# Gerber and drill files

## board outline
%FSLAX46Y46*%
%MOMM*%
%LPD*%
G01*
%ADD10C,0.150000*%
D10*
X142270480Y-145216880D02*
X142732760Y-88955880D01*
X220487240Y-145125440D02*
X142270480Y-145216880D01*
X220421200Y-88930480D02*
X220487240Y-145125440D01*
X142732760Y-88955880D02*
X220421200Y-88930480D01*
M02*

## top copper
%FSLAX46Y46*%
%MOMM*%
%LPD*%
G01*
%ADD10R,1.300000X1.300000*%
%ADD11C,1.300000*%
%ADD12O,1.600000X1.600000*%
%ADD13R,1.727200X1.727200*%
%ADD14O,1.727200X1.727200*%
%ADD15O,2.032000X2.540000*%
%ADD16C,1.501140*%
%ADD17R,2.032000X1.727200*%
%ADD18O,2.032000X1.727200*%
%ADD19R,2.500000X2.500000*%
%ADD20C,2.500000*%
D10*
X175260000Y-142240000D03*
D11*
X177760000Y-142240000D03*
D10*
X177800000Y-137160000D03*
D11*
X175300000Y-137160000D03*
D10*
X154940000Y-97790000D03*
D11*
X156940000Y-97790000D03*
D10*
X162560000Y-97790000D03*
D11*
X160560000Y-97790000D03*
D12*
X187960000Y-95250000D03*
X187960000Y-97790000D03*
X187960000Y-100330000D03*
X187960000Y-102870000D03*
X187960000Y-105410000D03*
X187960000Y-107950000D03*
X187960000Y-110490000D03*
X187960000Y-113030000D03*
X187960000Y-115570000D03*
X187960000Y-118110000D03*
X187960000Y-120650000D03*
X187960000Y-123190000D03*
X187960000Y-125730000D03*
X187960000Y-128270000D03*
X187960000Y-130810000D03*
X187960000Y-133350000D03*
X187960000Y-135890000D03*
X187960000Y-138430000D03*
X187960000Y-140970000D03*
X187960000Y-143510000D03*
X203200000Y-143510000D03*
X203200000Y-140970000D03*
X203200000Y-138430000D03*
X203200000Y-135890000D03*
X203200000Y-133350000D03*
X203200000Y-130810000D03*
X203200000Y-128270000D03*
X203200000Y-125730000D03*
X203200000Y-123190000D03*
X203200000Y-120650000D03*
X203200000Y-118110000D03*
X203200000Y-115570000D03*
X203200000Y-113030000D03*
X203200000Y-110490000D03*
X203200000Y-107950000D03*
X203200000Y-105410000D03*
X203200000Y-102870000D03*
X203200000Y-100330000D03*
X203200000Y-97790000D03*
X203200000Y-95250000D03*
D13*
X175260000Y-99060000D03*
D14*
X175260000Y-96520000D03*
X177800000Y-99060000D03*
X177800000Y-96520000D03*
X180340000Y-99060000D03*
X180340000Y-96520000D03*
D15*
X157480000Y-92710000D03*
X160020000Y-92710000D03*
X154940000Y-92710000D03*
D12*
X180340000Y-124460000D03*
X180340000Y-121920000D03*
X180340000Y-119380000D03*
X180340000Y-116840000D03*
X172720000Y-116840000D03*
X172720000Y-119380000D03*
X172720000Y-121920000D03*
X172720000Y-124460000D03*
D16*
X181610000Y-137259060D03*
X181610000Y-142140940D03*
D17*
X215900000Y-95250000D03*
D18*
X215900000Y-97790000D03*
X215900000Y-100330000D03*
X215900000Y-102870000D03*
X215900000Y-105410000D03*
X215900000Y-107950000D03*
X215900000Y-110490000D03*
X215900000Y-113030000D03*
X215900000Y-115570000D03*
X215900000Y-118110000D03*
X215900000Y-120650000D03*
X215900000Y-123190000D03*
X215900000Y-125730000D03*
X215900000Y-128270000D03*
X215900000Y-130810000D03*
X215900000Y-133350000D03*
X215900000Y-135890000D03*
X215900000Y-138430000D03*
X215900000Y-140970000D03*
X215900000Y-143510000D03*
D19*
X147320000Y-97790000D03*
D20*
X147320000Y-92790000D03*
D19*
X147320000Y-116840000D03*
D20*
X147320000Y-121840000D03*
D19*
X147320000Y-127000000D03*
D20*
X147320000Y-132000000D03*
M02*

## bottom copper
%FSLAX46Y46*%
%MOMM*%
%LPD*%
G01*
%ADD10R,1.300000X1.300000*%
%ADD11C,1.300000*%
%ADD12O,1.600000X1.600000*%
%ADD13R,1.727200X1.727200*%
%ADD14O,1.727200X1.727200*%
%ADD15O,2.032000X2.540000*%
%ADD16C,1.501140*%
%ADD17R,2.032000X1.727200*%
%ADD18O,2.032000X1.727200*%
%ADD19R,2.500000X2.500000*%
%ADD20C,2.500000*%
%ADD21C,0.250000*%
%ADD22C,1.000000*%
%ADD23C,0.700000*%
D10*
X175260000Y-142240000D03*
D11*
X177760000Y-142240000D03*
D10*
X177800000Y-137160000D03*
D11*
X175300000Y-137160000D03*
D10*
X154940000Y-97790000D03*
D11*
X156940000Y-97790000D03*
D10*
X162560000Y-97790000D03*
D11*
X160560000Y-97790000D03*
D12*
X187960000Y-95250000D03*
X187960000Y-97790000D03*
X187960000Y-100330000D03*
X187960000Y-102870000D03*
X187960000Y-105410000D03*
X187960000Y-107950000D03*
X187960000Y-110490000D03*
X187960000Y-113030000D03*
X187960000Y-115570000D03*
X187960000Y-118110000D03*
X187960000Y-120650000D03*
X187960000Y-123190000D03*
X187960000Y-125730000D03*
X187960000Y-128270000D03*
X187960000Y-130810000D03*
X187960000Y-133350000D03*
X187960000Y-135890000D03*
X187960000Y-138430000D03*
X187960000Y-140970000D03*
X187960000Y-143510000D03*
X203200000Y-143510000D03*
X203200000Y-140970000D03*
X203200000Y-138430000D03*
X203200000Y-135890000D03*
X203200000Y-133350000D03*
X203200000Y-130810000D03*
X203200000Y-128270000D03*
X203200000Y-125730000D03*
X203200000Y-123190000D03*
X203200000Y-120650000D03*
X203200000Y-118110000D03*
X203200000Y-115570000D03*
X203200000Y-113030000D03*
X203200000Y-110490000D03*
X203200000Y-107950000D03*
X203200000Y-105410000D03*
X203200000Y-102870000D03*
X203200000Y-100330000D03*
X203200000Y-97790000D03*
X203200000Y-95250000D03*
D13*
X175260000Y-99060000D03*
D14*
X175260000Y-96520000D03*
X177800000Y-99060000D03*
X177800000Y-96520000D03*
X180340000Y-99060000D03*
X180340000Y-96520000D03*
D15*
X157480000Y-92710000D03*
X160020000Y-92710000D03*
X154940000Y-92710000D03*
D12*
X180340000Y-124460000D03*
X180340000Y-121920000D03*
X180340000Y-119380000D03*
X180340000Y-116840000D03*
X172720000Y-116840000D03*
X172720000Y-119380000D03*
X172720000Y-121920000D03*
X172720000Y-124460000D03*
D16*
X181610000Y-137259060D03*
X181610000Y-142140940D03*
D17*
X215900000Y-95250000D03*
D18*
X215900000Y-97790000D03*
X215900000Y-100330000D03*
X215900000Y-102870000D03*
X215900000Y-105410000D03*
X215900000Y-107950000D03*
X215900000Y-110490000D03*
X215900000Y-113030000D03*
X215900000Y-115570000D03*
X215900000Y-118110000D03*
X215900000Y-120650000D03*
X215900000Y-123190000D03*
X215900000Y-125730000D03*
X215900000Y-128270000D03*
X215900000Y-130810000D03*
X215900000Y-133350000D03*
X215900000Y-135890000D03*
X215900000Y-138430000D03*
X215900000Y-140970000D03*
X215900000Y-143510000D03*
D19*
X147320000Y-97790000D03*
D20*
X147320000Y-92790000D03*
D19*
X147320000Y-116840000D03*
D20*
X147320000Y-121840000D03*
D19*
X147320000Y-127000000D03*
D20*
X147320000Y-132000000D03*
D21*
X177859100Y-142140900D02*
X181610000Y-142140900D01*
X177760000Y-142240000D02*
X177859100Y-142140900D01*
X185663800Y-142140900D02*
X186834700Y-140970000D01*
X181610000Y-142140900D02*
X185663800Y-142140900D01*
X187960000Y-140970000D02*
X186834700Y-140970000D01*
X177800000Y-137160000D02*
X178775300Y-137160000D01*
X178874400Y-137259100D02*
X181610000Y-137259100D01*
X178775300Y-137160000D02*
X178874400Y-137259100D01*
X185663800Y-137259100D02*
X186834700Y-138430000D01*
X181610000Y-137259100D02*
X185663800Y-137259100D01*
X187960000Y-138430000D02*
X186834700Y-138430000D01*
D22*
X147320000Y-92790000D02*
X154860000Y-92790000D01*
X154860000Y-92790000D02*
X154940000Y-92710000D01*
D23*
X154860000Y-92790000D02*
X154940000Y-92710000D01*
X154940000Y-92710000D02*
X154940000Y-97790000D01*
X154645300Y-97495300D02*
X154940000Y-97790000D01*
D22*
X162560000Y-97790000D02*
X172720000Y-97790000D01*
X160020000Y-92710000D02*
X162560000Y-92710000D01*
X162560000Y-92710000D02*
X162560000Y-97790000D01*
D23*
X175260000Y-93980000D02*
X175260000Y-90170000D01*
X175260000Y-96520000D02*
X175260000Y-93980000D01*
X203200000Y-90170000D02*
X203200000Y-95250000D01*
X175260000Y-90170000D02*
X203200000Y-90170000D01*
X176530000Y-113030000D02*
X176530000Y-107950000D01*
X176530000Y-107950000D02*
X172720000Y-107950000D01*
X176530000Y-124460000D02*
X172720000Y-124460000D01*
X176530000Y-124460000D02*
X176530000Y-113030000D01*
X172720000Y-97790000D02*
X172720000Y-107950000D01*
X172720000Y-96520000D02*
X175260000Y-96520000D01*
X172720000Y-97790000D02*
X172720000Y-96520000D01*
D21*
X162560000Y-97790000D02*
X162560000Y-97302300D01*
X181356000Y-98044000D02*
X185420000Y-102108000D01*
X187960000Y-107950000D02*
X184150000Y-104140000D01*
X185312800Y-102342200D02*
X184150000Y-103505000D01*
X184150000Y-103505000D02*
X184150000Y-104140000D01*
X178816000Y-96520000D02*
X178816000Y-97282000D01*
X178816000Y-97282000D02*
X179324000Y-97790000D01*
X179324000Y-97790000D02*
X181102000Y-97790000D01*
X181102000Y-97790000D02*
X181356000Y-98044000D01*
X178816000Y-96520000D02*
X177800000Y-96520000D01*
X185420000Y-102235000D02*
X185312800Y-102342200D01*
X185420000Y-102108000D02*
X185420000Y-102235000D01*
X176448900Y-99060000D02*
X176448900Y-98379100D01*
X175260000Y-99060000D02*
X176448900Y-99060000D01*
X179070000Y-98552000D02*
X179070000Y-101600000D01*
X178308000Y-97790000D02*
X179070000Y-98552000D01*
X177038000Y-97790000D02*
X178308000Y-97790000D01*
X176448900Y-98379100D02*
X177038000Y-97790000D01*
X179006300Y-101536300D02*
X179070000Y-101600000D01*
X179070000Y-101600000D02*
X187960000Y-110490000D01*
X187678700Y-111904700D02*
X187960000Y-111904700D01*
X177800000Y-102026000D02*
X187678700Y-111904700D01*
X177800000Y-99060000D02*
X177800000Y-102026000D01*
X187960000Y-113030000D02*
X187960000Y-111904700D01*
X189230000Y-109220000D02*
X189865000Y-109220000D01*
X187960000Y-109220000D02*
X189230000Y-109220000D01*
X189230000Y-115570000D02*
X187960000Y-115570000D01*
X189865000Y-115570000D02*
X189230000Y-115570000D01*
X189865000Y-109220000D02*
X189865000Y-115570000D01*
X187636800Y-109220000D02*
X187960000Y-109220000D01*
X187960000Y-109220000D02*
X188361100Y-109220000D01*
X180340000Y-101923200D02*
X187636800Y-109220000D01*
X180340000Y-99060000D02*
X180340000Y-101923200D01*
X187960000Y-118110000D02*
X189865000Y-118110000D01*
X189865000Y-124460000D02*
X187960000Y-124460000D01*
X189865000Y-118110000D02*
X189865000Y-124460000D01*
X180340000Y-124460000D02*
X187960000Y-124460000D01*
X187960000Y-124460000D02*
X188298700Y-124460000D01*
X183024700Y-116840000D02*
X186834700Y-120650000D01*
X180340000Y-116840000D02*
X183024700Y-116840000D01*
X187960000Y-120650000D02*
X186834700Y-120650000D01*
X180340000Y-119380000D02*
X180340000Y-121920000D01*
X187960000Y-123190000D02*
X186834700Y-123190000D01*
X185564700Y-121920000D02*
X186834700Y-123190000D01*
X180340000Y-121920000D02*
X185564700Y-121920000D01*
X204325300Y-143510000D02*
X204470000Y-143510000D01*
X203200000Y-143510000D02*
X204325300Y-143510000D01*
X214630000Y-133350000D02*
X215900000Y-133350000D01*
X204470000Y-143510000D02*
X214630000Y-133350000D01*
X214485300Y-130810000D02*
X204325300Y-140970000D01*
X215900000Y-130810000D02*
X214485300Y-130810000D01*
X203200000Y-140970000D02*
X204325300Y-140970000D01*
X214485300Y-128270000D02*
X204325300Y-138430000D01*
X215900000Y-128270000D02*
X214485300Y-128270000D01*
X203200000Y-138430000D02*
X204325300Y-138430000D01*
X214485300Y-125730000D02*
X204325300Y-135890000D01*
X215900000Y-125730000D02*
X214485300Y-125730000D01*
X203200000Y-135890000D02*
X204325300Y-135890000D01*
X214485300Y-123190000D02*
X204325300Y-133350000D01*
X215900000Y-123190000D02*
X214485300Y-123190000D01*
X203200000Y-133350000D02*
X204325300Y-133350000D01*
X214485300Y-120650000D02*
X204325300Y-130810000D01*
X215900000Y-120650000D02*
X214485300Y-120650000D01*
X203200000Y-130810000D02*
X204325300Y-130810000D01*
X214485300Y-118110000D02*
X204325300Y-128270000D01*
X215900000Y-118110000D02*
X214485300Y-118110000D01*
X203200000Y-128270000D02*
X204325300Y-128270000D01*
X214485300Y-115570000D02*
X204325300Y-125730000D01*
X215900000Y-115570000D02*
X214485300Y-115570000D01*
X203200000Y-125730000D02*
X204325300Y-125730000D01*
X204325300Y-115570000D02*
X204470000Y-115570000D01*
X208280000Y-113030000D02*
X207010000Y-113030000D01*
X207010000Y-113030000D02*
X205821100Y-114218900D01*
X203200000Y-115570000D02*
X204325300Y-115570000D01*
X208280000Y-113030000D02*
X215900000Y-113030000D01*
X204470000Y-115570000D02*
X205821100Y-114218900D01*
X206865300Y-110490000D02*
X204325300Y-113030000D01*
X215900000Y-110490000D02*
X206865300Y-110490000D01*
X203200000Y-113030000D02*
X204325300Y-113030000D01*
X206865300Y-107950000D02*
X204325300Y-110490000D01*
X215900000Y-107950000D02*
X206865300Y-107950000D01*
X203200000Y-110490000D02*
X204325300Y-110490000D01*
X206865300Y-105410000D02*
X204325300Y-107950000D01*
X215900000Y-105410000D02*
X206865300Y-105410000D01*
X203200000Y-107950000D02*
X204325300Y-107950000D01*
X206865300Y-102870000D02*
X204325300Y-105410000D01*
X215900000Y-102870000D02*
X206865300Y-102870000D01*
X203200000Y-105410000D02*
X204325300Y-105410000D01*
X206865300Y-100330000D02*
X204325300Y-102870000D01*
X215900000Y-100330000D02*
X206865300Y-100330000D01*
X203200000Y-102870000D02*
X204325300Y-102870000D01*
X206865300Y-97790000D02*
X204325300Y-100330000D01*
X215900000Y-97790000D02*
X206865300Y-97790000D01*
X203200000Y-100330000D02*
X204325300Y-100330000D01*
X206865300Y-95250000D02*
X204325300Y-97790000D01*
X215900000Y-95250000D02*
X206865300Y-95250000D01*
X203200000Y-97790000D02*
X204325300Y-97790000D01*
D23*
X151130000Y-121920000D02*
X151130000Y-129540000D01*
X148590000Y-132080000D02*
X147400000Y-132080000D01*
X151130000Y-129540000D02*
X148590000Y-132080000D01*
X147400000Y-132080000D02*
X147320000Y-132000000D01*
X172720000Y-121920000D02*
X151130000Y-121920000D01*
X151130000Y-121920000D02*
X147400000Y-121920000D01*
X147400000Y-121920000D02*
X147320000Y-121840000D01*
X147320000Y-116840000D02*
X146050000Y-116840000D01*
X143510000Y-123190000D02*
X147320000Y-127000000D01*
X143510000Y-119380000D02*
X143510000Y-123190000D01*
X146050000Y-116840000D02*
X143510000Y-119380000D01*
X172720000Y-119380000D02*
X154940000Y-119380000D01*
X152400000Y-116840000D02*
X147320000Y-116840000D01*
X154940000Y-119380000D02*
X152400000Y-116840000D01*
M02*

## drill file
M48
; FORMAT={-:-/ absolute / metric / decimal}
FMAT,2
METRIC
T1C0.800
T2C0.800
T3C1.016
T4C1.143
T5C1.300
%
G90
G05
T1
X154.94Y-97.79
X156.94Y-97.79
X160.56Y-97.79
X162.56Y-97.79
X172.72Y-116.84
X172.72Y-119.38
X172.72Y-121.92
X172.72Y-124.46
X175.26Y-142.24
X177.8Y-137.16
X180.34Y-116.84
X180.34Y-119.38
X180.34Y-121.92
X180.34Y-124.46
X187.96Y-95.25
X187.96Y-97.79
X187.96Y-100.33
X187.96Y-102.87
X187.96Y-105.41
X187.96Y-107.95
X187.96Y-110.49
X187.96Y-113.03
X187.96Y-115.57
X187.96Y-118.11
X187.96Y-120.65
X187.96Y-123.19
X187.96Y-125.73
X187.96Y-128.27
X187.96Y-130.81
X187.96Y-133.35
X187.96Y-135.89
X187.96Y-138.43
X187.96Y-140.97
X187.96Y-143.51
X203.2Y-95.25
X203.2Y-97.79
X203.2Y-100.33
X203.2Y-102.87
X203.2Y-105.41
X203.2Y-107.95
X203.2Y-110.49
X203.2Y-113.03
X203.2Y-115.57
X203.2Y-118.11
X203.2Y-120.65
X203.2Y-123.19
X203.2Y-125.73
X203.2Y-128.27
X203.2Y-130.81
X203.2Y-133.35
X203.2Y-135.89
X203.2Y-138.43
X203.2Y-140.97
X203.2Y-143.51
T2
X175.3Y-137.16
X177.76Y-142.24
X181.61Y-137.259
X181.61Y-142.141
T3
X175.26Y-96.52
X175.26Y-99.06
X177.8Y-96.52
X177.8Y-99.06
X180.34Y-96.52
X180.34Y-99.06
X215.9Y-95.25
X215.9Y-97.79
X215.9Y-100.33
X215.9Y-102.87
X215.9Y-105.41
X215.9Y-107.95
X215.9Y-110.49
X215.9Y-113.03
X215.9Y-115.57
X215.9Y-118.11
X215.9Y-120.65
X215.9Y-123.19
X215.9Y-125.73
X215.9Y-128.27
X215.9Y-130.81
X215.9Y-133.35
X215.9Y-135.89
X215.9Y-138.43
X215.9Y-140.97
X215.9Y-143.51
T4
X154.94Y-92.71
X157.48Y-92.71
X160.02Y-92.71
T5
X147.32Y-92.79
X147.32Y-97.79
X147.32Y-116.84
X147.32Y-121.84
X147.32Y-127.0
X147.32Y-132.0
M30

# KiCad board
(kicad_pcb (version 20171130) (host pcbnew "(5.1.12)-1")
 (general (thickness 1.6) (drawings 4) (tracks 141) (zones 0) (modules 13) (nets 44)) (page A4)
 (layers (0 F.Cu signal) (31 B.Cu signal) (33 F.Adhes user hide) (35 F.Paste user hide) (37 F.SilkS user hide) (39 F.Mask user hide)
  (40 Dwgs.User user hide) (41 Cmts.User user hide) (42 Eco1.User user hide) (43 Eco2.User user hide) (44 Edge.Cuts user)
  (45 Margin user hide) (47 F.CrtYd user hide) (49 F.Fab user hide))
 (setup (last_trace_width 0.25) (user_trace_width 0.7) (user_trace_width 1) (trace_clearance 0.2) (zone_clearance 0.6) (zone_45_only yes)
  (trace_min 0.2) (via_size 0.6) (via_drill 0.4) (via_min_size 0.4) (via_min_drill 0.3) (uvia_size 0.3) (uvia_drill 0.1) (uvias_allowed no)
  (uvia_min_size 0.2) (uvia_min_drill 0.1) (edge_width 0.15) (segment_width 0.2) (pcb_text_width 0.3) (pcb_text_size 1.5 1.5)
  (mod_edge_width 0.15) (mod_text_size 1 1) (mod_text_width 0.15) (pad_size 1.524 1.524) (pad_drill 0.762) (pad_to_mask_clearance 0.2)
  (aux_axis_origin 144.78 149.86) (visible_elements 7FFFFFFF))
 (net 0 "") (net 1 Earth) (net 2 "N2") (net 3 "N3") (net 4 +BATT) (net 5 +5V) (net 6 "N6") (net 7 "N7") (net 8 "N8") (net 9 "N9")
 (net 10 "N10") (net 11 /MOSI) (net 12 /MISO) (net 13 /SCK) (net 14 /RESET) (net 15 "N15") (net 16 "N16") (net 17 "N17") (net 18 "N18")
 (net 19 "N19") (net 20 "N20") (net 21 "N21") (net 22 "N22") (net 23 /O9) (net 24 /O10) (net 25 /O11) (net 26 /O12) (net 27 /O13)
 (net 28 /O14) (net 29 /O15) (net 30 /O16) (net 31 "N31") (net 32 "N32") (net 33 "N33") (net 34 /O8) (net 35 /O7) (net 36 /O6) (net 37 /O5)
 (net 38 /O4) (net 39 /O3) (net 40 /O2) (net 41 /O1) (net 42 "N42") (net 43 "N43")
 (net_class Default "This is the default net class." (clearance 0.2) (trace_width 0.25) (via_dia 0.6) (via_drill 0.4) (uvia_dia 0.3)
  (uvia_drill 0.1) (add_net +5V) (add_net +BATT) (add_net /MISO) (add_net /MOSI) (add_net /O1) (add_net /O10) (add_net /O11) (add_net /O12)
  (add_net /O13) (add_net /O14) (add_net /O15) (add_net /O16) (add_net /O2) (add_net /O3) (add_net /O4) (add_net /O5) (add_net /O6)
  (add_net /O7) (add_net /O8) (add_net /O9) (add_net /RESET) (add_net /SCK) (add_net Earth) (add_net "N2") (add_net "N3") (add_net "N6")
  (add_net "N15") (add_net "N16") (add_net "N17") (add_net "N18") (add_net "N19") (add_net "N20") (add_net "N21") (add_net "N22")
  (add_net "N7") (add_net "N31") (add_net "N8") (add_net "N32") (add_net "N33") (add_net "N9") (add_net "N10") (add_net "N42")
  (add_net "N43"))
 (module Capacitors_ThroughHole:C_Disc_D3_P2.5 (layer F.Cu) (at 175.26 142.24)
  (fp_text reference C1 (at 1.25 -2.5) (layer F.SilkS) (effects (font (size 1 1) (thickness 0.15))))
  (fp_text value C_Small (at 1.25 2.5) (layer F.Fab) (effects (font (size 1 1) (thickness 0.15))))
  (pad 1 thru_hole rect (at 0 0) (size 1.3 1.3) (drill 0.8) (layers *.Cu *.Mask F.SilkS) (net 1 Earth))
  (pad 2 thru_hole circle (at 2.5 0) (size 1.3 1.3) (drill 0.8001) (layers *.Cu *.Mask F.SilkS) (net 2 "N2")))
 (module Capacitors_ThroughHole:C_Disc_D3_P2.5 (layer F.Cu) (at 177.8 137.16 180)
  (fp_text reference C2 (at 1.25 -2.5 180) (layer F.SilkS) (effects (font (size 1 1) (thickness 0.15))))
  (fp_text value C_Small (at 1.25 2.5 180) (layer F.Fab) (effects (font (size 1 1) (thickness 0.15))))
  (pad 1 thru_hole rect (at 0 0 180) (size 1.3 1.3) (drill 0.8) (layers *.Cu *.Mask F.SilkS) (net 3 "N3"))
  (pad 2 thru_hole circle (at 2.5 0 180) (size 1.3 1.3) (drill 0.8001) (layers *.Cu *.Mask F.SilkS) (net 1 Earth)))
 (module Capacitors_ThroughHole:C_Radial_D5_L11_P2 (layer F.Cu) (at 154.94 97.79)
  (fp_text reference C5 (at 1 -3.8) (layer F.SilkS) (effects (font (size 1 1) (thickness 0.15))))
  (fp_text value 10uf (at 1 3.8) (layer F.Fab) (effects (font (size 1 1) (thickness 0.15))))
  (pad 1 thru_hole rect (at 0 0) (size 1.3 1.3) (drill 0.8) (layers *.Cu *.Mask F.SilkS) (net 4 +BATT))
  (pad 2 thru_hole circle (at 2 0) (size 1.3 1.3) (drill 0.8) (layers *.Cu *.Mask F.SilkS) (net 1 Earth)))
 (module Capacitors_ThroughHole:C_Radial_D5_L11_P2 (layer F.Cu) (at 162.56 97.79 180)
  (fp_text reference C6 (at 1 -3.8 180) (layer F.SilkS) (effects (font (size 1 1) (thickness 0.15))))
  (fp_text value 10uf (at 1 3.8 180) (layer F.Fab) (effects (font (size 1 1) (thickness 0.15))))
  (pad 1 thru_hole rect (at 0 0 180) (size 1.3 1.3) (drill 0.8) (layers *.Cu *.Mask F.SilkS) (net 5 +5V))
  (pad 2 thru_hole circle (at 2 0 180) (size 1.3 1.3) (drill 0.8) (layers *.Cu *.Mask F.SilkS) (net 1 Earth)))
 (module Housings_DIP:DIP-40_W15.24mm (layer F.Cu) (at 187.96 95.25)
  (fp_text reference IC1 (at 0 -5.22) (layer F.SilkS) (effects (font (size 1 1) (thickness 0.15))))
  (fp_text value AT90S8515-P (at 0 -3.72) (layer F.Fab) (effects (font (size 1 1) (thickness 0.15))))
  (pad 1 thru_hole oval (at 0 0) (size 1.6 1.6) (drill 0.8) (layers *.Cu *.Mask F.SilkS) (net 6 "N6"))
  (pad 2 thru_hole oval (at 0 2.54) (size 1.6 1.6) (drill 0.8) (layers *.Cu *.Mask F.SilkS) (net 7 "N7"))
  (pad 3 thru_hole oval (at 0 5.08) (size 1.6 1.6) (drill 0.8) (layers *.Cu *.Mask F.SilkS) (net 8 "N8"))
  (pad 4 thru_hole oval (at 0 7.62) (size 1.6 1.6) (drill 0.8) (layers *.Cu *.Mask F.SilkS) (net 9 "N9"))
  (pad 5 thru_hole oval (at 0 10.16) (size 1.6 1.6) (drill 0.8) (layers *.Cu *.Mask F.SilkS) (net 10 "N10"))
  (pad 6 thru_hole oval (at 0 12.7) (size 1.6 1.6) (drill 0.8) (layers *.Cu *.Mask F.SilkS) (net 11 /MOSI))
  (pad 7 thru_hole oval (at 0 15.24) (size 1.6 1.6) (drill 0.8) (layers *.Cu *.Mask F.SilkS) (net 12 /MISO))
  (pad 8 thru_hole oval (at 0 17.78) (size 1.6 1.6) (drill 0.8) (layers *.Cu *.Mask F.SilkS) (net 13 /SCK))
  (pad 9 thru_hole oval (at 0 20.32) (size 1.6 1.6) (drill 0.8) (layers *.Cu *.Mask F.SilkS) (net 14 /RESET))
  (pad 10 thru_hole oval (at 0 22.86) (size 1.6 1.6) (drill 0.8) (layers *.Cu *.Mask F.SilkS) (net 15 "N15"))
  (pad 11 thru_hole oval (at 0 25.4) (size 1.6 1.6) (drill 0.8) (layers *.Cu *.Mask F.SilkS) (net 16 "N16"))
  (pad 12 thru_hole oval (at 0 27.94) (size 1.6 1.6) (drill 0.8) (layers *.Cu *.Mask F.SilkS) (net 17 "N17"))
  (pad 13 thru_hole oval (at 0 30.48) (size 1.6 1.6) (drill 0.8) (layers *.Cu *.Mask F.SilkS) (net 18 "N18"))
  (pad 14 thru_hole oval (at 0 33.02) (size 1.6 1.6) (drill 0.8) (layers *.Cu *.Mask F.SilkS) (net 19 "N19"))
  (pad 15 thru_hole oval (at 0 35.56) (size 1.6 1.6) (drill 0.8) (layers *.Cu *.Mask F.SilkS) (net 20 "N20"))
  (pad 16 thru_hole oval (at 0 38.1) (size 1.6 1.6) (drill 0.8) (layers *.Cu *.Mask F.SilkS) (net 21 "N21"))
  (pad 17 thru_hole oval (at 0 40.64) (size 1.6 1.6) (drill 0.8) (layers *.Cu *.Mask F.SilkS) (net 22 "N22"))
  (pad 18 thru_hole oval (at 0 43.18) (size 1.6 1.6) (drill 0.8) (layers *.Cu *.Mask F.SilkS) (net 3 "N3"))
  (pad 19 thru_hole oval (at 0 45.72) (size 1.6 1.6) (drill 0.8) (layers *.Cu *.Mask F.SilkS) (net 2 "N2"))
  (pad 20 thru_hole oval (at 0 48.26) (size 1.6 1.6) (drill 0.8) (layers *.Cu *.Mask F.SilkS) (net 1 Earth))
  (pad 21 thru_hole oval (at 15.24 48.26) (size 1.6 1.6) (drill 0.8) (layers *.Cu *.Mask F.SilkS) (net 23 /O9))
  (pad 22 thru_hole oval (at 15.24 45.72) (size 1.6 1.6) (drill 0.8) (layers *.Cu *.Mask F.SilkS) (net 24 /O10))
  (pad 23 thru_hole oval (at 15.24 43.18) (size 1.6 1.6) (drill 0.8) (layers *.Cu *.Mask F.SilkS) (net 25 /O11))
  (pad 24 thru_hole oval (at 15.24 40.64) (size 1.6 1.6) (drill 0.8) (layers *.Cu *.Mask F.SilkS) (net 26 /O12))
  (pad 25 thru_hole oval (at 15.24 38.1) (size 1.6 1.6) (drill 0.8) (layers *.Cu *.Mask F.SilkS) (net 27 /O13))
  (pad 26 thru_hole oval (at 15.24 35.56) (size 1.6 1.6) (drill 0.8) (layers *.Cu *.Mask F.SilkS) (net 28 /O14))
  (pad 27 thru_hole oval (at 15.24 33.02) (size 1.6 1.6) (drill 0.8) (layers *.Cu *.Mask F.SilkS) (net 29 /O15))
  (pad 28 thru_hole oval (at 15.24 30.48) (size 1.6 1.6) (drill 0.8) (layers *.Cu *.Mask F.SilkS) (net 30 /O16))
  (pad 29 thru_hole oval (at 15.24 27.94) (size 1.6 1.6) (drill 0.8) (layers *.Cu *.Mask F.SilkS) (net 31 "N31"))
  (pad 30 thru_hole oval (at 15.24 25.4) (size 1.6 1.6) (drill 0.8) (layers *.Cu *.Mask F.SilkS) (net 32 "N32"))
  (pad 31 thru_hole oval (at 15.24 22.86) (size 1.6 1.6) (drill 0.8) (layers *.Cu *.Mask F.SilkS) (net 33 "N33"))
  (pad 32 thru_hole oval (at 15.24 20.32) (size 1.6 1.6) (drill 0.8) (layers *.Cu *.Mask F.SilkS) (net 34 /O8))
  (pad 33 thru_hole oval (at 15.24 17.78) (size 1.6 1.6) (drill 0.8) (layers *.Cu *.Mask F.SilkS) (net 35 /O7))
  (pad 34 thru_hole oval (at 15.24 15.24) (size 1.6 1.6) (drill 0.8) (layers *.Cu *.Mask F.SilkS) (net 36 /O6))
  (pad 35 thru_hole oval (at 15.24 12.7) (size 1.6 1.6) (drill 0.8) (layers *.Cu *.Mask F.SilkS) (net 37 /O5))
  (pad 36 thru_hole oval (at 15.24 10.16) (size 1.6 1.6) (drill 0.8) (layers *.Cu *.Mask F.SilkS) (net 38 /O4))
  (pad 37 thru_hole oval (at 15.24 7.62) (size 1.6 1.6) (drill 0.8) (layers *.Cu *.Mask F.SilkS) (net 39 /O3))
  (pad 38 thru_hole oval (at 15.24 5.08) (size 1.6 1.6) (drill 0.8) (layers *.Cu *.Mask F.SilkS) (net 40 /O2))
  (pad 39 thru_hole oval (at 15.24 2.54) (size 1.6 1.6) (drill 0.8) (layers *.Cu *.Mask F.SilkS) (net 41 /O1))
  (pad 40 thru_hole oval (at 15.24 0) (size 1.6 1.6) (drill 0.8) (layers *.Cu *.Mask F.SilkS) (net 5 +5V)))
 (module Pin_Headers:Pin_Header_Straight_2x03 (layer F.Cu) (at 175.26 99.06 90)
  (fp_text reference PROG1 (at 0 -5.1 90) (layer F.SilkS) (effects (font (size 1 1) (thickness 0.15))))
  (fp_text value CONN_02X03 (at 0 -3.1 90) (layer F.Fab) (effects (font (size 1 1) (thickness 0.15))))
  (pad 1 thru_hole rect (at 0 0 90) (size 1.7272 1.7272) (drill 1.016) (layers *.Cu *.Mask F.SilkS) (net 12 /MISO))
  (pad 2 thru_hole oval (at 2.54 0 90) (size 1.7272 1.7272) (drill 1.016) (layers *.Cu *.Mask F.SilkS) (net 5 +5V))
  (pad 3 thru_hole oval (at 0 2.54 90) (size 1.7272 1.7272) (drill 1.016) (layers *.Cu *.Mask F.SilkS) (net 13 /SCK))
  (pad 4 thru_hole oval (at 2.54 2.54 90) (size 1.7272 1.7272) (drill 1.016) (layers *.Cu *.Mask F.SilkS) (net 11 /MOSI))
  (pad 5 thru_hole oval (at 0 5.08 90) (size 1.7272 1.7272) (drill 1.016) (layers *.Cu *.Mask F.SilkS) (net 14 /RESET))
  (pad 6 thru_hole oval (at 2.54 5.08 90) (size 1.7272 1.7272) (drill 1.016) (layers *.Cu *.Mask F.SilkS) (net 1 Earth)))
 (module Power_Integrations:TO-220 (layer F.Cu) (at 157.48 92.71)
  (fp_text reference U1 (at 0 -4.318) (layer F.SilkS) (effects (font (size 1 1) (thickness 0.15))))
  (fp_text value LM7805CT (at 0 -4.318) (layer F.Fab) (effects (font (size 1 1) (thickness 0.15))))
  (pad 2 thru_hole oval (at 0 0) (size 2.032 2.54) (drill 1.143) (layers *.Cu *.Mask F.SilkS) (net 1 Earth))
  (pad 3 thru_hole oval (at 2.54 0) (size 2.032 2.54) (drill 1.143) (layers *.Cu *.Mask F.SilkS) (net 5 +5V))
  (pad 1 thru_hole oval (at -2.54 0) (size 2.032 2.54) (drill 1.143) (layers *.Cu *.Mask F.SilkS) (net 4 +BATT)))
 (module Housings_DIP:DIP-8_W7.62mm (layer F.Cu) (at 180.34 124.46 180)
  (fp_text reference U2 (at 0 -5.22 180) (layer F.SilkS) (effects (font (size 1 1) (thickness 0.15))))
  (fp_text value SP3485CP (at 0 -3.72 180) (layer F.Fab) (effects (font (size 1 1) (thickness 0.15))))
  (pad 1 thru_hole oval (at 0 0 180) (size 1.6 1.6) (drill 0.8) (layers *.Cu *.Mask F.SilkS) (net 15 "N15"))
  (pad 2 thru_hole oval (at 0 2.54 180) (size 1.6 1.6) (drill 0.8) (layers *.Cu *.Mask F.SilkS) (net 17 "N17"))
  (pad 3 thru_hole oval (at 0 5.08 180) (size 1.6 1.6) (drill 0.8) (layers *.Cu *.Mask F.SilkS) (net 17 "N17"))
  (pad 4 thru_hole oval (at 0 7.62 180) (size 1.6 1.6) (drill 0.8) (layers *.Cu *.Mask F.SilkS) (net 16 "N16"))
  (pad 5 thru_hole oval (at 7.62 7.62 180) (size 1.6 1.6) (drill 0.8) (layers *.Cu *.Mask F.SilkS) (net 1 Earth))
  (pad 6 thru_hole oval (at 7.62 5.08 180) (size 1.6 1.6) (drill 0.8) (layers *.Cu *.Mask F.SilkS) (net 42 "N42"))
  (pad 7 thru_hole oval (at 7.62 2.54 180) (size 1.6 1.6) (drill 0.8) (layers *.Cu *.Mask F.SilkS) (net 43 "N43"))
  (pad 8 thru_hole oval (at 7.62 0 180) (size 1.6 1.6) (drill 0.8) (layers *.Cu *.Mask F.SilkS) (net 5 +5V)))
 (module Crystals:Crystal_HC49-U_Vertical (layer F.Cu) (at 181.61 139.7 270)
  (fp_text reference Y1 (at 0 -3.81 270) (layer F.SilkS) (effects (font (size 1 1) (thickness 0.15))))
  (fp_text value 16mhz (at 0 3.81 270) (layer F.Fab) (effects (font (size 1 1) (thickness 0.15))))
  (pad 1 thru_hole circle (at -2.44094 0 270) (size 1.50114 1.50114) (drill 0.8001) (layers *.Cu *.Mask F.SilkS) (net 3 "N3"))
  (pad 2 thru_hole circle (at 2.44094 0 270) (size 1.50114 1.50114) (drill 0.8001) (layers *.Cu *.Mask F.SilkS) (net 2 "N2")))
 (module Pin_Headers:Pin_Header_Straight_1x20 (layer F.Cu) (at 215.9 95.25)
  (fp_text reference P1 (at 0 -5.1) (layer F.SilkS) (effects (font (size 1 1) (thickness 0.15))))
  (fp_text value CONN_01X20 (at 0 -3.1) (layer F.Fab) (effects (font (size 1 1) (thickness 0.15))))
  (pad 1 thru_hole rect (at 0 0) (size 2.032 1.7272) (drill 1.016) (layers *.Cu *.Mask F.SilkS) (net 41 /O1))
  (pad 2 thru_hole oval (at 0 2.54) (size 2.032 1.7272) (drill 1.016) (layers *.Cu *.Mask F.SilkS) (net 40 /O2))
  (pad 3 thru_hole oval (at 0 5.08) (size 2.032 1.7272) (drill 1.016) (layers *.Cu *.Mask F.SilkS) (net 39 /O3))
  (pad 4 thru_hole oval (at 0 7.62) (size 2.032 1.7272) (drill 1.016) (layers *.Cu *.Mask F.SilkS) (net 38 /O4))
  (pad 5 thru_hole oval (at 0 10.16) (size 2.032 1.7272) (drill 1.016) (layers *.Cu *.Mask F.SilkS) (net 37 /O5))
  (pad 6 thru_hole oval (at 0 12.7) (size 2.032 1.7272) (drill 1.016) (layers *.Cu *.Mask F.SilkS) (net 36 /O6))
  (pad 7 thru_hole oval (at 0 15.24) (size 2.032 1.7272) (drill 1.016) (layers *.Cu *.Mask F.SilkS) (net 35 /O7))
  (pad 8 thru_hole oval (at 0 17.78) (size 2.032 1.7272) (drill 1.016) (layers *.Cu *.Mask F.SilkS) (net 34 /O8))
  (pad 9 thru_hole oval (at 0 20.32) (size 2.032 1.7272) (drill 1.016) (layers *.Cu *.Mask F.SilkS) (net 30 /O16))
  (pad 10 thru_hole oval (at 0 22.86) (size 2.032 1.7272) (drill 1.016) (layers *.Cu *.Mask F.SilkS) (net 29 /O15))
  (pad 11 thru_hole oval (at 0 25.4) (size 2.032 1.7272) (drill 1.016) (layers *.Cu *.Mask F.SilkS) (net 28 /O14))
  (pad 12 thru_hole oval (at 0 27.94) (size 2.032 1.7272) (drill 1.016) (layers *.Cu *.Mask F.SilkS) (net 27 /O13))
  (pad 13 thru_hole oval (at 0 30.48) (size 2.032 1.7272) (drill 1.016) (layers *.Cu *.Mask F.SilkS) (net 26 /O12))
  (pad 14 thru_hole oval (at 0 33.02) (size 2.032 1.7272) (drill 1.016) (layers *.Cu *.Mask F.SilkS) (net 25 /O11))
  (pad 15 thru_hole oval (at 0 35.56) (size 2.032 1.7272) (drill 1.016) (layers *.Cu *.Mask F.SilkS) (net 24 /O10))
  (pad 16 thru_hole oval (at 0 38.1) (size 2.032 1.7272) (drill 1.016) (layers *.Cu *.Mask F.SilkS) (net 23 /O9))
  (pad 17 thru_hole oval (at 0 40.64) (size 2.032 1.7272) (drill 1.016) (layers *.Cu *.Mask F.SilkS) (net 1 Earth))
  (pad 18 thru_hole oval (at 0 43.18) (size 2.032 1.7272) (drill 1.016) (layers *.Cu *.Mask F.SilkS) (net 1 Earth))
  (pad 19 thru_hole oval (at 0 45.72) (size 2.032 1.7272) (drill 1.016) (layers *.Cu *.Mask F.SilkS) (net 1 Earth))
  (pad 20 thru_hole oval (at 0 48.26) (size 2.032 1.7272) (drill 1.016) (layers *.Cu *.Mask F.SilkS) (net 1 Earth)))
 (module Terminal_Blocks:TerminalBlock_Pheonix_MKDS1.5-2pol (layer F.Cu) (at 147.32 97.79 90)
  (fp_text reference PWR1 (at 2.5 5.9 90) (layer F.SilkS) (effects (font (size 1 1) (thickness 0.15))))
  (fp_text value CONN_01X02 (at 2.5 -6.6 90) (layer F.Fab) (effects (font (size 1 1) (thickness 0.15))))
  (pad 1 thru_hole rect (at 0 0 90) (size 2.5 2.5) (drill 1.3) (layers *.Cu *.Mask F.SilkS) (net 1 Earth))
  (pad 2 thru_hole circle (at 5 0 90) (size 2.5 2.5) (drill 1.3) (layers *.Cu *.Mask F.SilkS) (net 4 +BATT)))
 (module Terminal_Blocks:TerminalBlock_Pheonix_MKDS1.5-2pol (layer F.Cu) (at 147.32 116.84 270)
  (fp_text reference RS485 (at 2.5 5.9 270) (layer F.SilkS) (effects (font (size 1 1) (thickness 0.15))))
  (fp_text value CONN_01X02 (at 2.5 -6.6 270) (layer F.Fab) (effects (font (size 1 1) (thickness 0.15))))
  (pad 1 thru_hole rect (at 0 0 270) (size 2.5 2.5) (drill 1.3) (layers *.Cu *.Mask F.SilkS) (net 42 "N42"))
  (pad 2 thru_hole circle (at 5 0 270) (size 2.5 2.5) (drill 1.3) (layers *.Cu *.Mask F.SilkS) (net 43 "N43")))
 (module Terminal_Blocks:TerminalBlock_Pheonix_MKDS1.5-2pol (layer F.Cu) (at 147.32 127 270)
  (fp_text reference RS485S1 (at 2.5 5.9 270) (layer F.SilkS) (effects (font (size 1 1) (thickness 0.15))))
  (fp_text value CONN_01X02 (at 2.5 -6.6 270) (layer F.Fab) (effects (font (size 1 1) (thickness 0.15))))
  (pad 1 thru_hole rect (at 0 0 270) (size 2.5 2.5) (drill 1.3) (layers *.Cu *.Mask F.SilkS) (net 42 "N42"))
  (pad 2 thru_hole circle (at 5 0 270) (size 2.5 2.5) (drill 1.3) (layers *.Cu *.Mask F.SilkS) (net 43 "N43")))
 (gr_line (start 142.27048 145.21688) (end 142.73276 88.95588) (layer Edge.Cuts) (width 0.15))
 (gr_line (start 220.48724 145.12544) (end 142.27048 145.21688) (layer Edge.Cuts) (width 0.15))
 (gr_line (start 220.4212 88.93048) (end 220.48724 145.12544) (layer Edge.Cuts) (width 0.15))
 (gr_line (start 142.73276 88.95588) (end 220.4212 88.93048) (layer Edge.Cuts) (width 0.15))
 (segment (start 177.8591 142.1409) (end 181.61 142.1409) (width 0.25) (layer B.Cu) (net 2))
 (segment (start 177.76 142.24) (end 177.8591 142.1409) (width 0.25) (layer B.Cu) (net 2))
 (segment (start 185.6638 142.1409) (end 186.8347 140.97) (width 0.25) (layer B.Cu) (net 2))
 (segment (start 181.61 142.1409) (end 185.6638 142.1409) (width 0.25) (layer B.Cu) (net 2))
 (segment (start 187.96 140.97) (end 186.8347 140.97) (width 0.25) (layer B.Cu) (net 2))
 (segment (start 177.8 137.16) (end 178.7753 137.16) (width 0.25) (layer B.Cu) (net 3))
 (segment (start 178.8744 137.2591) (end 181.61 137.2591) (width 0.25) (layer B.Cu) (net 3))
 (segment (start 178.7753 137.16) (end 178.8744 137.2591) (width 0.25) (layer B.Cu) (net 3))
 (segment (start 185.6638 137.2591) (end 186.8347 138.43) (width 0.25) (layer B.Cu) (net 3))
 (segment (start 181.61 137.2591) (end 185.6638 137.2591) (width 0.25) (layer B.Cu) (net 3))
 (segment (start 187.96 138.43) (end 186.8347 138.43) (width 0.25) (layer B.Cu) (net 3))
 (segment (start 147.32 92.79) (end 154.86 92.79) (width 1) (layer B.Cu) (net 4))
 (segment (start 154.86 92.79) (end 154.94 92.71) (width 1) (layer B.Cu) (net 4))
 (segment (start 154.86 92.79) (end 154.94 92.71) (width 0.7) (layer B.Cu) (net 4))
 (segment (start 154.94 92.71) (end 154.94 97.79) (width 0.7) (layer B.Cu) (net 4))
 (segment (start 154.6453 97.4953) (end 154.94 97.79) (width 0.7) (layer B.Cu) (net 4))
 (segment (start 162.56 97.79) (end 172.72 97.79) (width 1) (layer B.Cu) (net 5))
 (segment (start 160.02 92.71) (end 162.56 92.71) (width 1) (layer B.Cu) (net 5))
 (segment (start 162.56 92.71) (end 162.56 97.79) (width 1) (layer B.Cu) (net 5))
 (segment (start 175.26 93.98) (end 175.26 90.17) (width 0.7) (layer B.Cu) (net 5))
 (segment (start 175.26 96.52) (end 175.26 93.98) (width 0.7) (layer B.Cu) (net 5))
 (segment (start 203.2 90.17) (end 203.2 95.25) (width 0.7) (layer B.Cu) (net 5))
 (segment (start 175.26 90.17) (end 203.2 90.17) (width 0.7) (layer B.Cu) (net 5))
 (segment (start 176.53 113.03) (end 176.53 107.95) (width 0.7) (layer B.Cu) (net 5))
 (segment (start 176.53 107.95) (end 172.72 107.95) (width 0.7) (layer B.Cu) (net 5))
 (segment (start 176.53 124.46) (end 172.72 124.46) (width 0.7) (layer B.Cu) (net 5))
 (segment (start 176.53 124.46) (end 176.53 113.03) (width 0.7) (layer B.Cu) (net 5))
 (segment (start 172.72 97.79) (end 172.72 107.95) (width 0.7) (layer B.Cu) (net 5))
 (segment (start 172.72 96.52) (end 175.26 96.52) (width 0.7) (layer B.Cu) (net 5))
 (segment (start 172.72 97.79) (end 172.72 96.52) (width 0.7) (layer B.Cu) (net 5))
 (segment (start 162.56 97.79) (end 162.56 97.3023) (width 0.25) (layer B.Cu) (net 5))
 (segment (start 181.356 98.044) (end 185.42 102.108) (width 0.25) (layer B.Cu) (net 11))
 (segment (start 187.96 107.95) (end 184.15 104.14) (width 0.25) (layer B.Cu) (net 11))
 (segment (start 185.3128 102.3422) (end 184.15 103.505) (width 0.25) (layer B.Cu) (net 11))
 (segment (start 184.15 103.505) (end 184.15 104.14) (width 0.25) (layer B.Cu) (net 11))
 (segment (start 178.816 96.52) (end 178.816 97.282) (width 0.25) (layer B.Cu) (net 11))
 (segment (start 178.816 97.282) (end 179.324 97.79) (width 0.25) (layer B.Cu) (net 11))
 (segment (start 179.324 97.79) (end 181.102 97.79) (width 0.25) (layer B.Cu) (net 11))
 (segment (start 181.102 97.79) (end 181.356 98.044) (width 0.25) (layer B.Cu) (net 11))
 (segment (start 178.816 96.52) (end 177.8 96.52) (width 0.25) (layer B.Cu) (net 11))
 (segment (start 185.42 102.235) (end 185.3128 102.3422) (width 0.25) (layer B.Cu) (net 11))
 (segment (start 185.42 102.108) (end 185.42 102.235) (width 0.25) (layer B.Cu) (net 11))
 (segment (start 176.4489 99.06) (end 176.4489 98.3791) (width 0.25) (layer B.Cu) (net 12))
 (segment (start 175.26 99.06) (end 176.4489 99.06) (width 0.25) (layer B.Cu) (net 12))
 (segment (start 179.07 98.552) (end 179.07 101.6) (width 0.25) (layer B.Cu) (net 12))
 (segment (start 178.308 97.79) (end 179.07 98.552) (width 0.25) (layer B.Cu) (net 12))
 (segment (start 177.038 97.79) (end 178.308 97.79) (width 0.25) (layer B.Cu) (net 12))
 (segment (start 176.4489 98.3791) (end 177.038 97.79) (width 0.25) (layer B.Cu) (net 12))
 (segment (start 179.0063 101.5363) (end 179.07 101.6) (width 0.25) (layer B.Cu) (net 12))
 (segment (start 179.07 101.6) (end 187.96 110.49) (width 0.25) (layer B.Cu) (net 12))
 (segment (start 187.6787 111.9047) (end 187.96 111.9047) (width 0.25) (layer B.Cu) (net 13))
 (segment (start 177.8 102.026) (end 187.6787 111.9047) (width 0.25) (layer B.Cu) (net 13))
 (segment (start 177.8 99.06) (end 177.8 102.026) (width 0.25) (layer B.Cu) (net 13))
 (segment (start 187.96 113.03) (end 187.96 111.9047) (width 0.25) (layer B.Cu) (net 13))
 (segment (start 189.23 109.22) (end 189.865 109.22) (width 0.25) (layer B.Cu) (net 14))
 (segment (start 187.96 109.22) (end 189.23 109.22) (width 0.25) (layer B.Cu) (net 14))
 (segment (start 189.23 115.57) (end 187.96 115.57) (width 0.25) (layer B.Cu) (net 14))
 (segment (start 189.865 115.57) (end 189.23 115.57) (width 0.25) (layer B.Cu) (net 14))
 (segment (start 189.865 109.22) (end 189.865 115.57) (width 0.25) (layer B.Cu) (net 14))
 (segment (start 187.6368 109.22) (end 187.96 109.22) (width 0.25) (layer B.Cu) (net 14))
 (segment (start 187.96 109.22) (end 188.3611 109.22) (width 0.25) (layer B.Cu) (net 14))
 (segment (start 180.34 101.9232) (end 187.6368 109.22) (width 0.25) (layer B.Cu) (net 14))
 (segment (start 180.34 99.06) (end 180.34 101.9232) (width 0.25) (layer B.Cu) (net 14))
 (segment (start 187.96 118.11) (end 189.865 118.11) (width 0.25) (layer B.Cu) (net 15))
 (segment (start 189.865 124.46) (end 187.96 124.46) (width 0.25) (layer B.Cu) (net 15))
 (segment (start 189.865 118.11) (end 189.865 124.46) (width 0.25) (layer B.Cu) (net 15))
 (segment (start 180.34 124.46) (end 187.96 124.46) (width 0.25) (layer B.Cu) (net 15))
 (segment (start 187.96 124.46) (end 188.2987 124.46) (width 0.25) (layer B.Cu) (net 15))
 (segment (start 183.0247 116.84) (end 186.8347 120.65) (width 0.25) (layer B.Cu) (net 16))
 (segment (start 180.34 116.84) (end 183.0247 116.84) (width 0.25) (layer B.Cu) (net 16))
 (segment (start 187.96 120.65) (end 186.8347 120.65) (width 0.25) (layer B.Cu) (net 16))
 (segment (start 180.34 119.38) (end 180.34 121.92) (width 0.25) (layer B.Cu) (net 17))
 (segment (start 187.96 123.19) (end 186.8347 123.19) (width 0.25) (layer B.Cu) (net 17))
 (segment (start 185.5647 121.92) (end 186.8347 123.19) (width 0.25) (layer B.Cu) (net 17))
 (segment (start 180.34 121.92) (end 185.5647 121.92) (width 0.25) (layer B.Cu) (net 17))
 (segment (start 204.3253 143.51) (end 204.47 143.51) (width 0.25) (layer B.Cu) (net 23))
 (segment (start 203.2 143.51) (end 204.3253 143.51) (width 0.25) (layer B.Cu) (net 23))
 (segment (start 214.63 133.35) (end 215.9 133.35) (width 0.25) (layer B.Cu) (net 23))
 (segment (start 204.47 143.51) (end 214.63 133.35) (width 0.25) (layer B.Cu) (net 23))
 (segment (start 214.4853 130.81) (end 204.3253 140.97) (width 0.25) (layer B.Cu) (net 24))
 (segment (start 215.9 130.81) (end 214.4853 130.81) (width 0.25) (layer B.Cu) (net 24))
 (segment (start 203.2 140.97) (end 204.3253 140.97) (width 0.25) (layer B.Cu) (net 24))
 (segment (start 214.4853 128.27) (end 204.3253 138.43) (width 0.25) (layer B.Cu) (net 25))
 (segment (start 215.9 128.27) (end 214.4853 128.27) (width 0.25) (layer B.Cu) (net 25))
 (segment (start 203.2 138.43) (end 204.3253 138.43) (width 0.25) (layer B.Cu) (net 25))
 (segment (start 214.4853 125.73) (end 204.3253 135.89) (width 0.25) (layer B.Cu) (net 26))
 (segment (start 215.9 125.73) (end 214.4853 125.73) (width 0.25) (layer B.Cu) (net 26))
 (segment (start 203.2 135.89) (end 204.3253 135.89) (width 0.25) (layer B.Cu) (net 26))
 (segment (start 214.4853 123.19) (end 204.3253 133.35) (width 0.25) (layer B.Cu) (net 27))
 (segment (start 215.9 123.19) (end 214.4853 123.19) (width 0.25) (layer B.Cu) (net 27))
 (segment (start 203.2 133.35) (end 204.3253 133.35) (width 0.25) (layer B.Cu) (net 27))
 (segment (start 214.4853 120.65) (end 204.3253 130.81) (width 0.25) (layer B.Cu) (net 28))
 (segment (start 215.9 120.65) (end 214.4853 120.65) (width 0.25) (layer B.Cu) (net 28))
 (segment (start 203.2 130.81) (end 204.3253 130.81) (width 0.25) (layer B.Cu) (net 28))
 (segment (start 214.4853 118.11) (end 204.3253 128.27) (width 0.25) (layer B.Cu) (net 29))
 (segment (start 215.9 118.11) (end 214.4853 118.11) (width 0.25) (layer B.Cu) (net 29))
 (segment (start 203.2 128.27) (end 204.3253 128.27) (width 0.25) (layer B.Cu) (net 29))
 (segment (start 214.4853 115.57) (end 204.3253 125.73) (width 0.25) (layer B.Cu) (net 30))
 (segment (start 215.9 115.57) (end 214.4853 115.57) (width 0.25) (layer B.Cu) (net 30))
 (segment (start 203.2 125.73) (end 204.3253 125.73) (width 0.25) (layer B.Cu) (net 30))
 (segment (start 204.3253 115.57) (end 204.47 115.57) (width 0.25) (layer B.Cu) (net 34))
 (segment (start 208.28 113.03) (end 207.01 113.03) (width 0.25) (layer B.Cu) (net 34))
 (segment (start 207.01 113.03) (end 205.8211 114.2189) (width 0.25) (layer B.Cu) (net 34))
 (segment (start 203.2 115.57) (end 204.3253 115.57) (width 0.25) (layer B.Cu) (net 34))
 (segment (start 208.28 113.03) (end 215.9 113.03) (width 0.25) (layer B.Cu) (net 34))
 (segment (start 204.47 115.57) (end 205.8211 114.2189) (width 0.25) (layer B.Cu) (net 34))
 (segment (start 206.8653 110.49) (end 204.3253 113.03) (width 0.25) (layer B.Cu) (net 35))
 (segment (start 215.9 110.49) (end 206.8653 110.49) (width 0.25) (layer B.Cu) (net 35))
 (segment (start 203.2 113.03) (end 204.3253 113.03) (width 0.25) (layer B.Cu) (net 35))
 (segment (start 206.8653 107.95) (end 204.3253 110.49) (width 0.25) (layer B.Cu) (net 36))
 (segment (start 215.9 107.95) (end 206.8653 107.95) (width 0.25) (layer B.Cu) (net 36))
 (segment (start 203.2 110.49) (end 204.3253 110.49) (width 0.25) (layer B.Cu) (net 36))
 (segment (start 206.8653 105.41) (end 204.3253 107.95) (width 0.25) (layer B.Cu) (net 37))
 (segment (start 215.9 105.41) (end 206.8653 105.41) (width 0.25) (layer B.Cu) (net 37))
 (segment (start 203.2 107.95) (end 204.3253 107.95) (width 0.25) (layer B.Cu) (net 37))
 (segment (start 206.8653 102.87) (end 204.3253 105.41) (width 0.25) (layer B.Cu) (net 38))
 (segment (start 215.9 102.87) (end 206.8653 102.87) (width 0.25) (layer B.Cu) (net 38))
 (segment (start 203.2 105.41) (end 204.3253 105.41) (width 0.25) (layer B.Cu) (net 38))
 (segment (start 206.8653 100.33) (end 204.3253 102.87) (width 0.25) (layer B.Cu) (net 39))
 (segment (start 215.9 100.33) (end 206.8653 100.33) (width 0.25) (layer B.Cu) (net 39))
 (segment (start 203.2 102.87) (end 204.3253 102.87) (width 0.25) (layer B.Cu) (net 39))
 (segment (start 206.8653 97.79) (end 204.3253 100.33) (width 0.25) (layer B.Cu) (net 40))
 (segment (start 215.9 97.79) (end 206.8653 97.79) (width 0.25) (layer B.Cu) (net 40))
 (segment (start 203.2 100.33) (end 204.3253 100.33) (width 0.25) (layer B.Cu) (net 40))
 (segment (start 206.8653 95.25) (end 204.3253 97.79) (width 0.25) (layer B.Cu) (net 41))
 (segment (start 215.9 95.25) (end 206.8653 95.25) (width 0.25) (layer B.Cu) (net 41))
 (segment (start 203.2 97.79) (end 204.3253 97.79) (width 0.25) (layer B.Cu) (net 41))
 (segment (start 151.13 121.92) (end 151.13 129.54) (width 0.7) (layer B.Cu) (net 43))
 (segment (start 148.59 132.08) (end 147.4 132.08) (width 0.7) (layer B.Cu) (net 43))
 (segment (start 151.13 129.54) (end 148.59 132.08) (width 0.7) (layer B.Cu) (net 43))
 (segment (start 147.4 132.08) (end 147.32 132) (width 0.7) (layer B.Cu) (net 43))
 (segment (start 172.72 121.92) (end 151.13 121.92) (width 0.7) (layer B.Cu) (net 43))
 (segment (start 151.13 121.92) (end 147.4 121.92) (width 0.7) (layer B.Cu) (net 43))
 (segment (start 147.4 121.92) (end 147.32 121.84) (width 0.7) (layer B.Cu) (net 43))
 (segment (start 147.32 116.84) (end 146.05 116.84) (width 0.7) (layer B.Cu) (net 42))
 (segment (start 143.51 123.19) (end 147.32 127) (width 0.7) (layer B.Cu) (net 42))
 (segment (start 143.51 119.38) (end 143.51 123.19) (width 0.7) (layer B.Cu) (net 42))
 (segment (start 146.05 116.84) (end 143.51 119.38) (width 0.7) (layer B.Cu) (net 42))
 (segment (start 172.72 119.38) (end 154.94 119.38) (width 0.7) (layer B.Cu) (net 42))
 (segment (start 152.4 116.84) (end 147.32 116.84) (width 0.7) (layer B.Cu) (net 42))
 (segment (start 154.94 119.38) (end 152.4 116.84) (width 0.7) (layer B.Cu) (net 42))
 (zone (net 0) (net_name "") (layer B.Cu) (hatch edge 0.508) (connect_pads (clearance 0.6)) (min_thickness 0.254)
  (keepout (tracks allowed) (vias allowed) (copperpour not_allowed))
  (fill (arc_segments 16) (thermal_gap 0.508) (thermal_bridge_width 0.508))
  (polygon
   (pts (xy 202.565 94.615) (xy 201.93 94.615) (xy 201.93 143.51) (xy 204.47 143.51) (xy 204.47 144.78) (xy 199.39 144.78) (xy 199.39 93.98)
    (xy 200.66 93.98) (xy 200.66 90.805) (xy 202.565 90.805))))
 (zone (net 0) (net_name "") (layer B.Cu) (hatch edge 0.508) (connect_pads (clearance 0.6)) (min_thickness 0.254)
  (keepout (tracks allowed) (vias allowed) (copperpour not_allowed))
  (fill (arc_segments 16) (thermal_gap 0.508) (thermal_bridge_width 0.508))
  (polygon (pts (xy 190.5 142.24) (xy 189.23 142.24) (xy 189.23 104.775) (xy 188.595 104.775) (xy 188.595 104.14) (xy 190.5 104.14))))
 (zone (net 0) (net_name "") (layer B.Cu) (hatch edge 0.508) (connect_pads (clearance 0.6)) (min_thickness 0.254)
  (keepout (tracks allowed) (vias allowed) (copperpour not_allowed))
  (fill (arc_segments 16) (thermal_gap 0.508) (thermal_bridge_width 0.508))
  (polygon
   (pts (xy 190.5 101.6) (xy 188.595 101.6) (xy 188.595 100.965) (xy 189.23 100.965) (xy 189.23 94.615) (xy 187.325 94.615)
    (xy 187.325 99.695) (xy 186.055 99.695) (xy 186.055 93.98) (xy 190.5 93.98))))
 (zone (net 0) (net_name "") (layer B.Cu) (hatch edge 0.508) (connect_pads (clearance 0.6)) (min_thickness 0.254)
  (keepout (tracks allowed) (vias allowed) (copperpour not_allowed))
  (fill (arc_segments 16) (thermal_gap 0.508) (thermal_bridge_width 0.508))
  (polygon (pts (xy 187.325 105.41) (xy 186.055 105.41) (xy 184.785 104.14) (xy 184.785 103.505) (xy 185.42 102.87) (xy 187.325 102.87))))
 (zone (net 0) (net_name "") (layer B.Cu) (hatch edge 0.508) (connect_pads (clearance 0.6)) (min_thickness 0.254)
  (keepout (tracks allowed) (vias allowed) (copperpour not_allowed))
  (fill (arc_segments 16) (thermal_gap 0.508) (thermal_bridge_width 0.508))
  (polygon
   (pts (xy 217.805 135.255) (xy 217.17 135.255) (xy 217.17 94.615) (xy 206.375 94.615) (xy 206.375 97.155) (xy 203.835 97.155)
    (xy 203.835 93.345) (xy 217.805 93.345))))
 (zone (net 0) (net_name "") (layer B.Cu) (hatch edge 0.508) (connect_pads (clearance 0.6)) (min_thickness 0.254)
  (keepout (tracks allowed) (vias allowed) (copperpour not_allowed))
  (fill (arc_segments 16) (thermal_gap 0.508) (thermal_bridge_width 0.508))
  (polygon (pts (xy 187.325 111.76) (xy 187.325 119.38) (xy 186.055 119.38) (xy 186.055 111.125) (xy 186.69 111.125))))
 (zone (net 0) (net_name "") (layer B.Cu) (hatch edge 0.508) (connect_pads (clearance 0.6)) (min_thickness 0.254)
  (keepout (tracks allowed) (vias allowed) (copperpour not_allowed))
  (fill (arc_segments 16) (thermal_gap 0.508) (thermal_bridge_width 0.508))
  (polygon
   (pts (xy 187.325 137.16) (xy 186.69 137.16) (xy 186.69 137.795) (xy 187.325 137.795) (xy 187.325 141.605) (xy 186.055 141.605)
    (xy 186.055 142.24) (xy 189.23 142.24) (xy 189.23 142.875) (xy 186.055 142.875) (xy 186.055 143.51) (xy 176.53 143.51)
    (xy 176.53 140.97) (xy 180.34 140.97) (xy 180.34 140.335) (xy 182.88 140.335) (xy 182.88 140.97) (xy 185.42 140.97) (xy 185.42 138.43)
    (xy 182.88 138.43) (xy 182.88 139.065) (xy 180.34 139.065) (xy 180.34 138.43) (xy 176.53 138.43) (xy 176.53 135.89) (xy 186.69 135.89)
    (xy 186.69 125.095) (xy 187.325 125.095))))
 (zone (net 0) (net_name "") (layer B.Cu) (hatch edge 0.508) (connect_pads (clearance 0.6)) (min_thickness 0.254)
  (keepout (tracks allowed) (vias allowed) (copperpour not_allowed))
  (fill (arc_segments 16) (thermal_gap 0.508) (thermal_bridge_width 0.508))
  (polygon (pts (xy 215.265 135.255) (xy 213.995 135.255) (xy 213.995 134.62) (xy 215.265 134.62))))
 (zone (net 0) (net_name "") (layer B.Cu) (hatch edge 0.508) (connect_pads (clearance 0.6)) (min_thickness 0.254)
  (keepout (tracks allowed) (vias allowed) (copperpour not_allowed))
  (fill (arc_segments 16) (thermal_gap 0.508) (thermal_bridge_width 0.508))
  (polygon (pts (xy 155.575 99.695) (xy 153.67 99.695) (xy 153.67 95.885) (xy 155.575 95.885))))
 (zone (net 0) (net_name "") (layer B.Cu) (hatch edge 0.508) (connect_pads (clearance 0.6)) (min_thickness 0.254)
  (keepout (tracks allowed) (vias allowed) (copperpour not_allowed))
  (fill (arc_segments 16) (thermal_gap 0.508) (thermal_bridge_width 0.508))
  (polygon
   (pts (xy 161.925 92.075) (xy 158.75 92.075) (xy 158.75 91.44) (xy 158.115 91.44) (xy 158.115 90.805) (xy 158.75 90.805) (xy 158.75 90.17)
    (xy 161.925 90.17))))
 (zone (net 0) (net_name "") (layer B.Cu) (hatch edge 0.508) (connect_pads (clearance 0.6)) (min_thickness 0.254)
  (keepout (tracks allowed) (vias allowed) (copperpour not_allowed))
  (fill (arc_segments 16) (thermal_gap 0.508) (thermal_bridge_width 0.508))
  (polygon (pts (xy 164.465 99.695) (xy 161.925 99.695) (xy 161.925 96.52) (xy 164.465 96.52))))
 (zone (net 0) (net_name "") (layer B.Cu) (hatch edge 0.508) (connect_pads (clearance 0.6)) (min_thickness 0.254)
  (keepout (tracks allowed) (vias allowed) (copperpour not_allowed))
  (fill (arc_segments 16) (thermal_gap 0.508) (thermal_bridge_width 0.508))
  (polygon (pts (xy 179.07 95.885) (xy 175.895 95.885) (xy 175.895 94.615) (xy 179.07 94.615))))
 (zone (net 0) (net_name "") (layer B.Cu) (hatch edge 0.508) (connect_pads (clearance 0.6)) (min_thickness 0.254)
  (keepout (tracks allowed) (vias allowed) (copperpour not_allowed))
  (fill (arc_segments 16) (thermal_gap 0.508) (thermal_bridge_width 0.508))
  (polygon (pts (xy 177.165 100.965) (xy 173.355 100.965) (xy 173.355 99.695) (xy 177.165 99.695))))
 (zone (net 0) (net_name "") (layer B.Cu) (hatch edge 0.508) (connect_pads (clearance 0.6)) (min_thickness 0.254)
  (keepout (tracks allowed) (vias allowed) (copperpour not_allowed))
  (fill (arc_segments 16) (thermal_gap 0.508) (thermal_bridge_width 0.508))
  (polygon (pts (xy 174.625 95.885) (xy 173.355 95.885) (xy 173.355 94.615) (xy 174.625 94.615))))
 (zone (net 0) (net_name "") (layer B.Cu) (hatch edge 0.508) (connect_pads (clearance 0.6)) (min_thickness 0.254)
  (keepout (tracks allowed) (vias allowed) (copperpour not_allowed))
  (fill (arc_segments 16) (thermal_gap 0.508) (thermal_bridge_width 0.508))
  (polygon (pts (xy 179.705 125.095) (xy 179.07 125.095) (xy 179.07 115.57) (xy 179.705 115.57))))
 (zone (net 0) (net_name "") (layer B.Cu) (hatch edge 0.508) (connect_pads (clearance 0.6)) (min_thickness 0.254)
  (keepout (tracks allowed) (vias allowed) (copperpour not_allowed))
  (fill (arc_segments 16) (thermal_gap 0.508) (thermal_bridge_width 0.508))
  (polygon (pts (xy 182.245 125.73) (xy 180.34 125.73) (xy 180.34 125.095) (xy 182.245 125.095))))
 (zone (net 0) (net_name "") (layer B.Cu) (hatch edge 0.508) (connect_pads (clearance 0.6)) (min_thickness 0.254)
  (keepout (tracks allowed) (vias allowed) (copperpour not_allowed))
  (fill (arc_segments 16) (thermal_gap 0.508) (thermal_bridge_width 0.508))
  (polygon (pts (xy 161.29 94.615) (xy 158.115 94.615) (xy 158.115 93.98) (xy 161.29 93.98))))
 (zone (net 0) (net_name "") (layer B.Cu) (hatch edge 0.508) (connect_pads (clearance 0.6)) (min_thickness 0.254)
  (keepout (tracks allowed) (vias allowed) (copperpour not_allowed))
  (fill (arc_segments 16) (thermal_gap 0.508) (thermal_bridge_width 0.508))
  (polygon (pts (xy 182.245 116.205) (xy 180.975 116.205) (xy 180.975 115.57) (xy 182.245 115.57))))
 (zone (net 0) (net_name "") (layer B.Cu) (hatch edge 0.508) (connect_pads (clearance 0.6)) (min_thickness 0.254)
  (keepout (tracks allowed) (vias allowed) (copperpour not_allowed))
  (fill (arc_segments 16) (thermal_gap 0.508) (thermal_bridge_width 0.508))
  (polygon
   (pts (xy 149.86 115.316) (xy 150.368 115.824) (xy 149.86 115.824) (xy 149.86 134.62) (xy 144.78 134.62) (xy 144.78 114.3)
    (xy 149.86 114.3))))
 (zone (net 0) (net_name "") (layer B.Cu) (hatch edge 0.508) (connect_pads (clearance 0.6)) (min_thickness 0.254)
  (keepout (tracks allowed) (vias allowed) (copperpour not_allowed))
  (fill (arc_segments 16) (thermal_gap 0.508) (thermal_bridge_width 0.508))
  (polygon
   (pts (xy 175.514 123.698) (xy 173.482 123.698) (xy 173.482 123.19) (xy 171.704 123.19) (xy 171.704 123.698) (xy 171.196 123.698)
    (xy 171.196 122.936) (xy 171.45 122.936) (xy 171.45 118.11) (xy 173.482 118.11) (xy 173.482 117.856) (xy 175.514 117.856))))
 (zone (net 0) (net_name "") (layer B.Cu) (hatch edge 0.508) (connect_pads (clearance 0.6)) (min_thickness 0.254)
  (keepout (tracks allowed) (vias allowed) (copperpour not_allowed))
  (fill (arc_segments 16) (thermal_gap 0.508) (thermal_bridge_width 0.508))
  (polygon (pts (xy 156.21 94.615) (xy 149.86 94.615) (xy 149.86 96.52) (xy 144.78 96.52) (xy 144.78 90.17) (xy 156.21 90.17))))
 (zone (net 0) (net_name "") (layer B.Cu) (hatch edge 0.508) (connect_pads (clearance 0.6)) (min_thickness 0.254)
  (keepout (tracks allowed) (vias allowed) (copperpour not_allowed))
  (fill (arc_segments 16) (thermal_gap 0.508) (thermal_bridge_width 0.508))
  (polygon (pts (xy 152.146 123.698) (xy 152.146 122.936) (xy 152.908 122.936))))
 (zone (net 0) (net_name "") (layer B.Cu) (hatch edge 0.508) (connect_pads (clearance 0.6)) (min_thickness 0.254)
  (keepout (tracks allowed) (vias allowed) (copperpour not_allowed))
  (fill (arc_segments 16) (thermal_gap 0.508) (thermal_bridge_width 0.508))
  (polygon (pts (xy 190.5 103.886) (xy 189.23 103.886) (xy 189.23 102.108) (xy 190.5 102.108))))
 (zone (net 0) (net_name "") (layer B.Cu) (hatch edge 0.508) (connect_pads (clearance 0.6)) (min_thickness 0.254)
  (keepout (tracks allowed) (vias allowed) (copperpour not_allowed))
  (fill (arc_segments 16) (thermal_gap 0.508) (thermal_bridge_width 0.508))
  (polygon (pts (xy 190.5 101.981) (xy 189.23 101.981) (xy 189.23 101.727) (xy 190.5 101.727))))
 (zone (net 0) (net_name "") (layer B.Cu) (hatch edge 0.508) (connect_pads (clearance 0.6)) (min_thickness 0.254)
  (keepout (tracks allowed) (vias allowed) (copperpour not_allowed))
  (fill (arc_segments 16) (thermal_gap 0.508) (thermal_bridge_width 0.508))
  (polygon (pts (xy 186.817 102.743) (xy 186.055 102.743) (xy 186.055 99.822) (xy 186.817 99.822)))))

